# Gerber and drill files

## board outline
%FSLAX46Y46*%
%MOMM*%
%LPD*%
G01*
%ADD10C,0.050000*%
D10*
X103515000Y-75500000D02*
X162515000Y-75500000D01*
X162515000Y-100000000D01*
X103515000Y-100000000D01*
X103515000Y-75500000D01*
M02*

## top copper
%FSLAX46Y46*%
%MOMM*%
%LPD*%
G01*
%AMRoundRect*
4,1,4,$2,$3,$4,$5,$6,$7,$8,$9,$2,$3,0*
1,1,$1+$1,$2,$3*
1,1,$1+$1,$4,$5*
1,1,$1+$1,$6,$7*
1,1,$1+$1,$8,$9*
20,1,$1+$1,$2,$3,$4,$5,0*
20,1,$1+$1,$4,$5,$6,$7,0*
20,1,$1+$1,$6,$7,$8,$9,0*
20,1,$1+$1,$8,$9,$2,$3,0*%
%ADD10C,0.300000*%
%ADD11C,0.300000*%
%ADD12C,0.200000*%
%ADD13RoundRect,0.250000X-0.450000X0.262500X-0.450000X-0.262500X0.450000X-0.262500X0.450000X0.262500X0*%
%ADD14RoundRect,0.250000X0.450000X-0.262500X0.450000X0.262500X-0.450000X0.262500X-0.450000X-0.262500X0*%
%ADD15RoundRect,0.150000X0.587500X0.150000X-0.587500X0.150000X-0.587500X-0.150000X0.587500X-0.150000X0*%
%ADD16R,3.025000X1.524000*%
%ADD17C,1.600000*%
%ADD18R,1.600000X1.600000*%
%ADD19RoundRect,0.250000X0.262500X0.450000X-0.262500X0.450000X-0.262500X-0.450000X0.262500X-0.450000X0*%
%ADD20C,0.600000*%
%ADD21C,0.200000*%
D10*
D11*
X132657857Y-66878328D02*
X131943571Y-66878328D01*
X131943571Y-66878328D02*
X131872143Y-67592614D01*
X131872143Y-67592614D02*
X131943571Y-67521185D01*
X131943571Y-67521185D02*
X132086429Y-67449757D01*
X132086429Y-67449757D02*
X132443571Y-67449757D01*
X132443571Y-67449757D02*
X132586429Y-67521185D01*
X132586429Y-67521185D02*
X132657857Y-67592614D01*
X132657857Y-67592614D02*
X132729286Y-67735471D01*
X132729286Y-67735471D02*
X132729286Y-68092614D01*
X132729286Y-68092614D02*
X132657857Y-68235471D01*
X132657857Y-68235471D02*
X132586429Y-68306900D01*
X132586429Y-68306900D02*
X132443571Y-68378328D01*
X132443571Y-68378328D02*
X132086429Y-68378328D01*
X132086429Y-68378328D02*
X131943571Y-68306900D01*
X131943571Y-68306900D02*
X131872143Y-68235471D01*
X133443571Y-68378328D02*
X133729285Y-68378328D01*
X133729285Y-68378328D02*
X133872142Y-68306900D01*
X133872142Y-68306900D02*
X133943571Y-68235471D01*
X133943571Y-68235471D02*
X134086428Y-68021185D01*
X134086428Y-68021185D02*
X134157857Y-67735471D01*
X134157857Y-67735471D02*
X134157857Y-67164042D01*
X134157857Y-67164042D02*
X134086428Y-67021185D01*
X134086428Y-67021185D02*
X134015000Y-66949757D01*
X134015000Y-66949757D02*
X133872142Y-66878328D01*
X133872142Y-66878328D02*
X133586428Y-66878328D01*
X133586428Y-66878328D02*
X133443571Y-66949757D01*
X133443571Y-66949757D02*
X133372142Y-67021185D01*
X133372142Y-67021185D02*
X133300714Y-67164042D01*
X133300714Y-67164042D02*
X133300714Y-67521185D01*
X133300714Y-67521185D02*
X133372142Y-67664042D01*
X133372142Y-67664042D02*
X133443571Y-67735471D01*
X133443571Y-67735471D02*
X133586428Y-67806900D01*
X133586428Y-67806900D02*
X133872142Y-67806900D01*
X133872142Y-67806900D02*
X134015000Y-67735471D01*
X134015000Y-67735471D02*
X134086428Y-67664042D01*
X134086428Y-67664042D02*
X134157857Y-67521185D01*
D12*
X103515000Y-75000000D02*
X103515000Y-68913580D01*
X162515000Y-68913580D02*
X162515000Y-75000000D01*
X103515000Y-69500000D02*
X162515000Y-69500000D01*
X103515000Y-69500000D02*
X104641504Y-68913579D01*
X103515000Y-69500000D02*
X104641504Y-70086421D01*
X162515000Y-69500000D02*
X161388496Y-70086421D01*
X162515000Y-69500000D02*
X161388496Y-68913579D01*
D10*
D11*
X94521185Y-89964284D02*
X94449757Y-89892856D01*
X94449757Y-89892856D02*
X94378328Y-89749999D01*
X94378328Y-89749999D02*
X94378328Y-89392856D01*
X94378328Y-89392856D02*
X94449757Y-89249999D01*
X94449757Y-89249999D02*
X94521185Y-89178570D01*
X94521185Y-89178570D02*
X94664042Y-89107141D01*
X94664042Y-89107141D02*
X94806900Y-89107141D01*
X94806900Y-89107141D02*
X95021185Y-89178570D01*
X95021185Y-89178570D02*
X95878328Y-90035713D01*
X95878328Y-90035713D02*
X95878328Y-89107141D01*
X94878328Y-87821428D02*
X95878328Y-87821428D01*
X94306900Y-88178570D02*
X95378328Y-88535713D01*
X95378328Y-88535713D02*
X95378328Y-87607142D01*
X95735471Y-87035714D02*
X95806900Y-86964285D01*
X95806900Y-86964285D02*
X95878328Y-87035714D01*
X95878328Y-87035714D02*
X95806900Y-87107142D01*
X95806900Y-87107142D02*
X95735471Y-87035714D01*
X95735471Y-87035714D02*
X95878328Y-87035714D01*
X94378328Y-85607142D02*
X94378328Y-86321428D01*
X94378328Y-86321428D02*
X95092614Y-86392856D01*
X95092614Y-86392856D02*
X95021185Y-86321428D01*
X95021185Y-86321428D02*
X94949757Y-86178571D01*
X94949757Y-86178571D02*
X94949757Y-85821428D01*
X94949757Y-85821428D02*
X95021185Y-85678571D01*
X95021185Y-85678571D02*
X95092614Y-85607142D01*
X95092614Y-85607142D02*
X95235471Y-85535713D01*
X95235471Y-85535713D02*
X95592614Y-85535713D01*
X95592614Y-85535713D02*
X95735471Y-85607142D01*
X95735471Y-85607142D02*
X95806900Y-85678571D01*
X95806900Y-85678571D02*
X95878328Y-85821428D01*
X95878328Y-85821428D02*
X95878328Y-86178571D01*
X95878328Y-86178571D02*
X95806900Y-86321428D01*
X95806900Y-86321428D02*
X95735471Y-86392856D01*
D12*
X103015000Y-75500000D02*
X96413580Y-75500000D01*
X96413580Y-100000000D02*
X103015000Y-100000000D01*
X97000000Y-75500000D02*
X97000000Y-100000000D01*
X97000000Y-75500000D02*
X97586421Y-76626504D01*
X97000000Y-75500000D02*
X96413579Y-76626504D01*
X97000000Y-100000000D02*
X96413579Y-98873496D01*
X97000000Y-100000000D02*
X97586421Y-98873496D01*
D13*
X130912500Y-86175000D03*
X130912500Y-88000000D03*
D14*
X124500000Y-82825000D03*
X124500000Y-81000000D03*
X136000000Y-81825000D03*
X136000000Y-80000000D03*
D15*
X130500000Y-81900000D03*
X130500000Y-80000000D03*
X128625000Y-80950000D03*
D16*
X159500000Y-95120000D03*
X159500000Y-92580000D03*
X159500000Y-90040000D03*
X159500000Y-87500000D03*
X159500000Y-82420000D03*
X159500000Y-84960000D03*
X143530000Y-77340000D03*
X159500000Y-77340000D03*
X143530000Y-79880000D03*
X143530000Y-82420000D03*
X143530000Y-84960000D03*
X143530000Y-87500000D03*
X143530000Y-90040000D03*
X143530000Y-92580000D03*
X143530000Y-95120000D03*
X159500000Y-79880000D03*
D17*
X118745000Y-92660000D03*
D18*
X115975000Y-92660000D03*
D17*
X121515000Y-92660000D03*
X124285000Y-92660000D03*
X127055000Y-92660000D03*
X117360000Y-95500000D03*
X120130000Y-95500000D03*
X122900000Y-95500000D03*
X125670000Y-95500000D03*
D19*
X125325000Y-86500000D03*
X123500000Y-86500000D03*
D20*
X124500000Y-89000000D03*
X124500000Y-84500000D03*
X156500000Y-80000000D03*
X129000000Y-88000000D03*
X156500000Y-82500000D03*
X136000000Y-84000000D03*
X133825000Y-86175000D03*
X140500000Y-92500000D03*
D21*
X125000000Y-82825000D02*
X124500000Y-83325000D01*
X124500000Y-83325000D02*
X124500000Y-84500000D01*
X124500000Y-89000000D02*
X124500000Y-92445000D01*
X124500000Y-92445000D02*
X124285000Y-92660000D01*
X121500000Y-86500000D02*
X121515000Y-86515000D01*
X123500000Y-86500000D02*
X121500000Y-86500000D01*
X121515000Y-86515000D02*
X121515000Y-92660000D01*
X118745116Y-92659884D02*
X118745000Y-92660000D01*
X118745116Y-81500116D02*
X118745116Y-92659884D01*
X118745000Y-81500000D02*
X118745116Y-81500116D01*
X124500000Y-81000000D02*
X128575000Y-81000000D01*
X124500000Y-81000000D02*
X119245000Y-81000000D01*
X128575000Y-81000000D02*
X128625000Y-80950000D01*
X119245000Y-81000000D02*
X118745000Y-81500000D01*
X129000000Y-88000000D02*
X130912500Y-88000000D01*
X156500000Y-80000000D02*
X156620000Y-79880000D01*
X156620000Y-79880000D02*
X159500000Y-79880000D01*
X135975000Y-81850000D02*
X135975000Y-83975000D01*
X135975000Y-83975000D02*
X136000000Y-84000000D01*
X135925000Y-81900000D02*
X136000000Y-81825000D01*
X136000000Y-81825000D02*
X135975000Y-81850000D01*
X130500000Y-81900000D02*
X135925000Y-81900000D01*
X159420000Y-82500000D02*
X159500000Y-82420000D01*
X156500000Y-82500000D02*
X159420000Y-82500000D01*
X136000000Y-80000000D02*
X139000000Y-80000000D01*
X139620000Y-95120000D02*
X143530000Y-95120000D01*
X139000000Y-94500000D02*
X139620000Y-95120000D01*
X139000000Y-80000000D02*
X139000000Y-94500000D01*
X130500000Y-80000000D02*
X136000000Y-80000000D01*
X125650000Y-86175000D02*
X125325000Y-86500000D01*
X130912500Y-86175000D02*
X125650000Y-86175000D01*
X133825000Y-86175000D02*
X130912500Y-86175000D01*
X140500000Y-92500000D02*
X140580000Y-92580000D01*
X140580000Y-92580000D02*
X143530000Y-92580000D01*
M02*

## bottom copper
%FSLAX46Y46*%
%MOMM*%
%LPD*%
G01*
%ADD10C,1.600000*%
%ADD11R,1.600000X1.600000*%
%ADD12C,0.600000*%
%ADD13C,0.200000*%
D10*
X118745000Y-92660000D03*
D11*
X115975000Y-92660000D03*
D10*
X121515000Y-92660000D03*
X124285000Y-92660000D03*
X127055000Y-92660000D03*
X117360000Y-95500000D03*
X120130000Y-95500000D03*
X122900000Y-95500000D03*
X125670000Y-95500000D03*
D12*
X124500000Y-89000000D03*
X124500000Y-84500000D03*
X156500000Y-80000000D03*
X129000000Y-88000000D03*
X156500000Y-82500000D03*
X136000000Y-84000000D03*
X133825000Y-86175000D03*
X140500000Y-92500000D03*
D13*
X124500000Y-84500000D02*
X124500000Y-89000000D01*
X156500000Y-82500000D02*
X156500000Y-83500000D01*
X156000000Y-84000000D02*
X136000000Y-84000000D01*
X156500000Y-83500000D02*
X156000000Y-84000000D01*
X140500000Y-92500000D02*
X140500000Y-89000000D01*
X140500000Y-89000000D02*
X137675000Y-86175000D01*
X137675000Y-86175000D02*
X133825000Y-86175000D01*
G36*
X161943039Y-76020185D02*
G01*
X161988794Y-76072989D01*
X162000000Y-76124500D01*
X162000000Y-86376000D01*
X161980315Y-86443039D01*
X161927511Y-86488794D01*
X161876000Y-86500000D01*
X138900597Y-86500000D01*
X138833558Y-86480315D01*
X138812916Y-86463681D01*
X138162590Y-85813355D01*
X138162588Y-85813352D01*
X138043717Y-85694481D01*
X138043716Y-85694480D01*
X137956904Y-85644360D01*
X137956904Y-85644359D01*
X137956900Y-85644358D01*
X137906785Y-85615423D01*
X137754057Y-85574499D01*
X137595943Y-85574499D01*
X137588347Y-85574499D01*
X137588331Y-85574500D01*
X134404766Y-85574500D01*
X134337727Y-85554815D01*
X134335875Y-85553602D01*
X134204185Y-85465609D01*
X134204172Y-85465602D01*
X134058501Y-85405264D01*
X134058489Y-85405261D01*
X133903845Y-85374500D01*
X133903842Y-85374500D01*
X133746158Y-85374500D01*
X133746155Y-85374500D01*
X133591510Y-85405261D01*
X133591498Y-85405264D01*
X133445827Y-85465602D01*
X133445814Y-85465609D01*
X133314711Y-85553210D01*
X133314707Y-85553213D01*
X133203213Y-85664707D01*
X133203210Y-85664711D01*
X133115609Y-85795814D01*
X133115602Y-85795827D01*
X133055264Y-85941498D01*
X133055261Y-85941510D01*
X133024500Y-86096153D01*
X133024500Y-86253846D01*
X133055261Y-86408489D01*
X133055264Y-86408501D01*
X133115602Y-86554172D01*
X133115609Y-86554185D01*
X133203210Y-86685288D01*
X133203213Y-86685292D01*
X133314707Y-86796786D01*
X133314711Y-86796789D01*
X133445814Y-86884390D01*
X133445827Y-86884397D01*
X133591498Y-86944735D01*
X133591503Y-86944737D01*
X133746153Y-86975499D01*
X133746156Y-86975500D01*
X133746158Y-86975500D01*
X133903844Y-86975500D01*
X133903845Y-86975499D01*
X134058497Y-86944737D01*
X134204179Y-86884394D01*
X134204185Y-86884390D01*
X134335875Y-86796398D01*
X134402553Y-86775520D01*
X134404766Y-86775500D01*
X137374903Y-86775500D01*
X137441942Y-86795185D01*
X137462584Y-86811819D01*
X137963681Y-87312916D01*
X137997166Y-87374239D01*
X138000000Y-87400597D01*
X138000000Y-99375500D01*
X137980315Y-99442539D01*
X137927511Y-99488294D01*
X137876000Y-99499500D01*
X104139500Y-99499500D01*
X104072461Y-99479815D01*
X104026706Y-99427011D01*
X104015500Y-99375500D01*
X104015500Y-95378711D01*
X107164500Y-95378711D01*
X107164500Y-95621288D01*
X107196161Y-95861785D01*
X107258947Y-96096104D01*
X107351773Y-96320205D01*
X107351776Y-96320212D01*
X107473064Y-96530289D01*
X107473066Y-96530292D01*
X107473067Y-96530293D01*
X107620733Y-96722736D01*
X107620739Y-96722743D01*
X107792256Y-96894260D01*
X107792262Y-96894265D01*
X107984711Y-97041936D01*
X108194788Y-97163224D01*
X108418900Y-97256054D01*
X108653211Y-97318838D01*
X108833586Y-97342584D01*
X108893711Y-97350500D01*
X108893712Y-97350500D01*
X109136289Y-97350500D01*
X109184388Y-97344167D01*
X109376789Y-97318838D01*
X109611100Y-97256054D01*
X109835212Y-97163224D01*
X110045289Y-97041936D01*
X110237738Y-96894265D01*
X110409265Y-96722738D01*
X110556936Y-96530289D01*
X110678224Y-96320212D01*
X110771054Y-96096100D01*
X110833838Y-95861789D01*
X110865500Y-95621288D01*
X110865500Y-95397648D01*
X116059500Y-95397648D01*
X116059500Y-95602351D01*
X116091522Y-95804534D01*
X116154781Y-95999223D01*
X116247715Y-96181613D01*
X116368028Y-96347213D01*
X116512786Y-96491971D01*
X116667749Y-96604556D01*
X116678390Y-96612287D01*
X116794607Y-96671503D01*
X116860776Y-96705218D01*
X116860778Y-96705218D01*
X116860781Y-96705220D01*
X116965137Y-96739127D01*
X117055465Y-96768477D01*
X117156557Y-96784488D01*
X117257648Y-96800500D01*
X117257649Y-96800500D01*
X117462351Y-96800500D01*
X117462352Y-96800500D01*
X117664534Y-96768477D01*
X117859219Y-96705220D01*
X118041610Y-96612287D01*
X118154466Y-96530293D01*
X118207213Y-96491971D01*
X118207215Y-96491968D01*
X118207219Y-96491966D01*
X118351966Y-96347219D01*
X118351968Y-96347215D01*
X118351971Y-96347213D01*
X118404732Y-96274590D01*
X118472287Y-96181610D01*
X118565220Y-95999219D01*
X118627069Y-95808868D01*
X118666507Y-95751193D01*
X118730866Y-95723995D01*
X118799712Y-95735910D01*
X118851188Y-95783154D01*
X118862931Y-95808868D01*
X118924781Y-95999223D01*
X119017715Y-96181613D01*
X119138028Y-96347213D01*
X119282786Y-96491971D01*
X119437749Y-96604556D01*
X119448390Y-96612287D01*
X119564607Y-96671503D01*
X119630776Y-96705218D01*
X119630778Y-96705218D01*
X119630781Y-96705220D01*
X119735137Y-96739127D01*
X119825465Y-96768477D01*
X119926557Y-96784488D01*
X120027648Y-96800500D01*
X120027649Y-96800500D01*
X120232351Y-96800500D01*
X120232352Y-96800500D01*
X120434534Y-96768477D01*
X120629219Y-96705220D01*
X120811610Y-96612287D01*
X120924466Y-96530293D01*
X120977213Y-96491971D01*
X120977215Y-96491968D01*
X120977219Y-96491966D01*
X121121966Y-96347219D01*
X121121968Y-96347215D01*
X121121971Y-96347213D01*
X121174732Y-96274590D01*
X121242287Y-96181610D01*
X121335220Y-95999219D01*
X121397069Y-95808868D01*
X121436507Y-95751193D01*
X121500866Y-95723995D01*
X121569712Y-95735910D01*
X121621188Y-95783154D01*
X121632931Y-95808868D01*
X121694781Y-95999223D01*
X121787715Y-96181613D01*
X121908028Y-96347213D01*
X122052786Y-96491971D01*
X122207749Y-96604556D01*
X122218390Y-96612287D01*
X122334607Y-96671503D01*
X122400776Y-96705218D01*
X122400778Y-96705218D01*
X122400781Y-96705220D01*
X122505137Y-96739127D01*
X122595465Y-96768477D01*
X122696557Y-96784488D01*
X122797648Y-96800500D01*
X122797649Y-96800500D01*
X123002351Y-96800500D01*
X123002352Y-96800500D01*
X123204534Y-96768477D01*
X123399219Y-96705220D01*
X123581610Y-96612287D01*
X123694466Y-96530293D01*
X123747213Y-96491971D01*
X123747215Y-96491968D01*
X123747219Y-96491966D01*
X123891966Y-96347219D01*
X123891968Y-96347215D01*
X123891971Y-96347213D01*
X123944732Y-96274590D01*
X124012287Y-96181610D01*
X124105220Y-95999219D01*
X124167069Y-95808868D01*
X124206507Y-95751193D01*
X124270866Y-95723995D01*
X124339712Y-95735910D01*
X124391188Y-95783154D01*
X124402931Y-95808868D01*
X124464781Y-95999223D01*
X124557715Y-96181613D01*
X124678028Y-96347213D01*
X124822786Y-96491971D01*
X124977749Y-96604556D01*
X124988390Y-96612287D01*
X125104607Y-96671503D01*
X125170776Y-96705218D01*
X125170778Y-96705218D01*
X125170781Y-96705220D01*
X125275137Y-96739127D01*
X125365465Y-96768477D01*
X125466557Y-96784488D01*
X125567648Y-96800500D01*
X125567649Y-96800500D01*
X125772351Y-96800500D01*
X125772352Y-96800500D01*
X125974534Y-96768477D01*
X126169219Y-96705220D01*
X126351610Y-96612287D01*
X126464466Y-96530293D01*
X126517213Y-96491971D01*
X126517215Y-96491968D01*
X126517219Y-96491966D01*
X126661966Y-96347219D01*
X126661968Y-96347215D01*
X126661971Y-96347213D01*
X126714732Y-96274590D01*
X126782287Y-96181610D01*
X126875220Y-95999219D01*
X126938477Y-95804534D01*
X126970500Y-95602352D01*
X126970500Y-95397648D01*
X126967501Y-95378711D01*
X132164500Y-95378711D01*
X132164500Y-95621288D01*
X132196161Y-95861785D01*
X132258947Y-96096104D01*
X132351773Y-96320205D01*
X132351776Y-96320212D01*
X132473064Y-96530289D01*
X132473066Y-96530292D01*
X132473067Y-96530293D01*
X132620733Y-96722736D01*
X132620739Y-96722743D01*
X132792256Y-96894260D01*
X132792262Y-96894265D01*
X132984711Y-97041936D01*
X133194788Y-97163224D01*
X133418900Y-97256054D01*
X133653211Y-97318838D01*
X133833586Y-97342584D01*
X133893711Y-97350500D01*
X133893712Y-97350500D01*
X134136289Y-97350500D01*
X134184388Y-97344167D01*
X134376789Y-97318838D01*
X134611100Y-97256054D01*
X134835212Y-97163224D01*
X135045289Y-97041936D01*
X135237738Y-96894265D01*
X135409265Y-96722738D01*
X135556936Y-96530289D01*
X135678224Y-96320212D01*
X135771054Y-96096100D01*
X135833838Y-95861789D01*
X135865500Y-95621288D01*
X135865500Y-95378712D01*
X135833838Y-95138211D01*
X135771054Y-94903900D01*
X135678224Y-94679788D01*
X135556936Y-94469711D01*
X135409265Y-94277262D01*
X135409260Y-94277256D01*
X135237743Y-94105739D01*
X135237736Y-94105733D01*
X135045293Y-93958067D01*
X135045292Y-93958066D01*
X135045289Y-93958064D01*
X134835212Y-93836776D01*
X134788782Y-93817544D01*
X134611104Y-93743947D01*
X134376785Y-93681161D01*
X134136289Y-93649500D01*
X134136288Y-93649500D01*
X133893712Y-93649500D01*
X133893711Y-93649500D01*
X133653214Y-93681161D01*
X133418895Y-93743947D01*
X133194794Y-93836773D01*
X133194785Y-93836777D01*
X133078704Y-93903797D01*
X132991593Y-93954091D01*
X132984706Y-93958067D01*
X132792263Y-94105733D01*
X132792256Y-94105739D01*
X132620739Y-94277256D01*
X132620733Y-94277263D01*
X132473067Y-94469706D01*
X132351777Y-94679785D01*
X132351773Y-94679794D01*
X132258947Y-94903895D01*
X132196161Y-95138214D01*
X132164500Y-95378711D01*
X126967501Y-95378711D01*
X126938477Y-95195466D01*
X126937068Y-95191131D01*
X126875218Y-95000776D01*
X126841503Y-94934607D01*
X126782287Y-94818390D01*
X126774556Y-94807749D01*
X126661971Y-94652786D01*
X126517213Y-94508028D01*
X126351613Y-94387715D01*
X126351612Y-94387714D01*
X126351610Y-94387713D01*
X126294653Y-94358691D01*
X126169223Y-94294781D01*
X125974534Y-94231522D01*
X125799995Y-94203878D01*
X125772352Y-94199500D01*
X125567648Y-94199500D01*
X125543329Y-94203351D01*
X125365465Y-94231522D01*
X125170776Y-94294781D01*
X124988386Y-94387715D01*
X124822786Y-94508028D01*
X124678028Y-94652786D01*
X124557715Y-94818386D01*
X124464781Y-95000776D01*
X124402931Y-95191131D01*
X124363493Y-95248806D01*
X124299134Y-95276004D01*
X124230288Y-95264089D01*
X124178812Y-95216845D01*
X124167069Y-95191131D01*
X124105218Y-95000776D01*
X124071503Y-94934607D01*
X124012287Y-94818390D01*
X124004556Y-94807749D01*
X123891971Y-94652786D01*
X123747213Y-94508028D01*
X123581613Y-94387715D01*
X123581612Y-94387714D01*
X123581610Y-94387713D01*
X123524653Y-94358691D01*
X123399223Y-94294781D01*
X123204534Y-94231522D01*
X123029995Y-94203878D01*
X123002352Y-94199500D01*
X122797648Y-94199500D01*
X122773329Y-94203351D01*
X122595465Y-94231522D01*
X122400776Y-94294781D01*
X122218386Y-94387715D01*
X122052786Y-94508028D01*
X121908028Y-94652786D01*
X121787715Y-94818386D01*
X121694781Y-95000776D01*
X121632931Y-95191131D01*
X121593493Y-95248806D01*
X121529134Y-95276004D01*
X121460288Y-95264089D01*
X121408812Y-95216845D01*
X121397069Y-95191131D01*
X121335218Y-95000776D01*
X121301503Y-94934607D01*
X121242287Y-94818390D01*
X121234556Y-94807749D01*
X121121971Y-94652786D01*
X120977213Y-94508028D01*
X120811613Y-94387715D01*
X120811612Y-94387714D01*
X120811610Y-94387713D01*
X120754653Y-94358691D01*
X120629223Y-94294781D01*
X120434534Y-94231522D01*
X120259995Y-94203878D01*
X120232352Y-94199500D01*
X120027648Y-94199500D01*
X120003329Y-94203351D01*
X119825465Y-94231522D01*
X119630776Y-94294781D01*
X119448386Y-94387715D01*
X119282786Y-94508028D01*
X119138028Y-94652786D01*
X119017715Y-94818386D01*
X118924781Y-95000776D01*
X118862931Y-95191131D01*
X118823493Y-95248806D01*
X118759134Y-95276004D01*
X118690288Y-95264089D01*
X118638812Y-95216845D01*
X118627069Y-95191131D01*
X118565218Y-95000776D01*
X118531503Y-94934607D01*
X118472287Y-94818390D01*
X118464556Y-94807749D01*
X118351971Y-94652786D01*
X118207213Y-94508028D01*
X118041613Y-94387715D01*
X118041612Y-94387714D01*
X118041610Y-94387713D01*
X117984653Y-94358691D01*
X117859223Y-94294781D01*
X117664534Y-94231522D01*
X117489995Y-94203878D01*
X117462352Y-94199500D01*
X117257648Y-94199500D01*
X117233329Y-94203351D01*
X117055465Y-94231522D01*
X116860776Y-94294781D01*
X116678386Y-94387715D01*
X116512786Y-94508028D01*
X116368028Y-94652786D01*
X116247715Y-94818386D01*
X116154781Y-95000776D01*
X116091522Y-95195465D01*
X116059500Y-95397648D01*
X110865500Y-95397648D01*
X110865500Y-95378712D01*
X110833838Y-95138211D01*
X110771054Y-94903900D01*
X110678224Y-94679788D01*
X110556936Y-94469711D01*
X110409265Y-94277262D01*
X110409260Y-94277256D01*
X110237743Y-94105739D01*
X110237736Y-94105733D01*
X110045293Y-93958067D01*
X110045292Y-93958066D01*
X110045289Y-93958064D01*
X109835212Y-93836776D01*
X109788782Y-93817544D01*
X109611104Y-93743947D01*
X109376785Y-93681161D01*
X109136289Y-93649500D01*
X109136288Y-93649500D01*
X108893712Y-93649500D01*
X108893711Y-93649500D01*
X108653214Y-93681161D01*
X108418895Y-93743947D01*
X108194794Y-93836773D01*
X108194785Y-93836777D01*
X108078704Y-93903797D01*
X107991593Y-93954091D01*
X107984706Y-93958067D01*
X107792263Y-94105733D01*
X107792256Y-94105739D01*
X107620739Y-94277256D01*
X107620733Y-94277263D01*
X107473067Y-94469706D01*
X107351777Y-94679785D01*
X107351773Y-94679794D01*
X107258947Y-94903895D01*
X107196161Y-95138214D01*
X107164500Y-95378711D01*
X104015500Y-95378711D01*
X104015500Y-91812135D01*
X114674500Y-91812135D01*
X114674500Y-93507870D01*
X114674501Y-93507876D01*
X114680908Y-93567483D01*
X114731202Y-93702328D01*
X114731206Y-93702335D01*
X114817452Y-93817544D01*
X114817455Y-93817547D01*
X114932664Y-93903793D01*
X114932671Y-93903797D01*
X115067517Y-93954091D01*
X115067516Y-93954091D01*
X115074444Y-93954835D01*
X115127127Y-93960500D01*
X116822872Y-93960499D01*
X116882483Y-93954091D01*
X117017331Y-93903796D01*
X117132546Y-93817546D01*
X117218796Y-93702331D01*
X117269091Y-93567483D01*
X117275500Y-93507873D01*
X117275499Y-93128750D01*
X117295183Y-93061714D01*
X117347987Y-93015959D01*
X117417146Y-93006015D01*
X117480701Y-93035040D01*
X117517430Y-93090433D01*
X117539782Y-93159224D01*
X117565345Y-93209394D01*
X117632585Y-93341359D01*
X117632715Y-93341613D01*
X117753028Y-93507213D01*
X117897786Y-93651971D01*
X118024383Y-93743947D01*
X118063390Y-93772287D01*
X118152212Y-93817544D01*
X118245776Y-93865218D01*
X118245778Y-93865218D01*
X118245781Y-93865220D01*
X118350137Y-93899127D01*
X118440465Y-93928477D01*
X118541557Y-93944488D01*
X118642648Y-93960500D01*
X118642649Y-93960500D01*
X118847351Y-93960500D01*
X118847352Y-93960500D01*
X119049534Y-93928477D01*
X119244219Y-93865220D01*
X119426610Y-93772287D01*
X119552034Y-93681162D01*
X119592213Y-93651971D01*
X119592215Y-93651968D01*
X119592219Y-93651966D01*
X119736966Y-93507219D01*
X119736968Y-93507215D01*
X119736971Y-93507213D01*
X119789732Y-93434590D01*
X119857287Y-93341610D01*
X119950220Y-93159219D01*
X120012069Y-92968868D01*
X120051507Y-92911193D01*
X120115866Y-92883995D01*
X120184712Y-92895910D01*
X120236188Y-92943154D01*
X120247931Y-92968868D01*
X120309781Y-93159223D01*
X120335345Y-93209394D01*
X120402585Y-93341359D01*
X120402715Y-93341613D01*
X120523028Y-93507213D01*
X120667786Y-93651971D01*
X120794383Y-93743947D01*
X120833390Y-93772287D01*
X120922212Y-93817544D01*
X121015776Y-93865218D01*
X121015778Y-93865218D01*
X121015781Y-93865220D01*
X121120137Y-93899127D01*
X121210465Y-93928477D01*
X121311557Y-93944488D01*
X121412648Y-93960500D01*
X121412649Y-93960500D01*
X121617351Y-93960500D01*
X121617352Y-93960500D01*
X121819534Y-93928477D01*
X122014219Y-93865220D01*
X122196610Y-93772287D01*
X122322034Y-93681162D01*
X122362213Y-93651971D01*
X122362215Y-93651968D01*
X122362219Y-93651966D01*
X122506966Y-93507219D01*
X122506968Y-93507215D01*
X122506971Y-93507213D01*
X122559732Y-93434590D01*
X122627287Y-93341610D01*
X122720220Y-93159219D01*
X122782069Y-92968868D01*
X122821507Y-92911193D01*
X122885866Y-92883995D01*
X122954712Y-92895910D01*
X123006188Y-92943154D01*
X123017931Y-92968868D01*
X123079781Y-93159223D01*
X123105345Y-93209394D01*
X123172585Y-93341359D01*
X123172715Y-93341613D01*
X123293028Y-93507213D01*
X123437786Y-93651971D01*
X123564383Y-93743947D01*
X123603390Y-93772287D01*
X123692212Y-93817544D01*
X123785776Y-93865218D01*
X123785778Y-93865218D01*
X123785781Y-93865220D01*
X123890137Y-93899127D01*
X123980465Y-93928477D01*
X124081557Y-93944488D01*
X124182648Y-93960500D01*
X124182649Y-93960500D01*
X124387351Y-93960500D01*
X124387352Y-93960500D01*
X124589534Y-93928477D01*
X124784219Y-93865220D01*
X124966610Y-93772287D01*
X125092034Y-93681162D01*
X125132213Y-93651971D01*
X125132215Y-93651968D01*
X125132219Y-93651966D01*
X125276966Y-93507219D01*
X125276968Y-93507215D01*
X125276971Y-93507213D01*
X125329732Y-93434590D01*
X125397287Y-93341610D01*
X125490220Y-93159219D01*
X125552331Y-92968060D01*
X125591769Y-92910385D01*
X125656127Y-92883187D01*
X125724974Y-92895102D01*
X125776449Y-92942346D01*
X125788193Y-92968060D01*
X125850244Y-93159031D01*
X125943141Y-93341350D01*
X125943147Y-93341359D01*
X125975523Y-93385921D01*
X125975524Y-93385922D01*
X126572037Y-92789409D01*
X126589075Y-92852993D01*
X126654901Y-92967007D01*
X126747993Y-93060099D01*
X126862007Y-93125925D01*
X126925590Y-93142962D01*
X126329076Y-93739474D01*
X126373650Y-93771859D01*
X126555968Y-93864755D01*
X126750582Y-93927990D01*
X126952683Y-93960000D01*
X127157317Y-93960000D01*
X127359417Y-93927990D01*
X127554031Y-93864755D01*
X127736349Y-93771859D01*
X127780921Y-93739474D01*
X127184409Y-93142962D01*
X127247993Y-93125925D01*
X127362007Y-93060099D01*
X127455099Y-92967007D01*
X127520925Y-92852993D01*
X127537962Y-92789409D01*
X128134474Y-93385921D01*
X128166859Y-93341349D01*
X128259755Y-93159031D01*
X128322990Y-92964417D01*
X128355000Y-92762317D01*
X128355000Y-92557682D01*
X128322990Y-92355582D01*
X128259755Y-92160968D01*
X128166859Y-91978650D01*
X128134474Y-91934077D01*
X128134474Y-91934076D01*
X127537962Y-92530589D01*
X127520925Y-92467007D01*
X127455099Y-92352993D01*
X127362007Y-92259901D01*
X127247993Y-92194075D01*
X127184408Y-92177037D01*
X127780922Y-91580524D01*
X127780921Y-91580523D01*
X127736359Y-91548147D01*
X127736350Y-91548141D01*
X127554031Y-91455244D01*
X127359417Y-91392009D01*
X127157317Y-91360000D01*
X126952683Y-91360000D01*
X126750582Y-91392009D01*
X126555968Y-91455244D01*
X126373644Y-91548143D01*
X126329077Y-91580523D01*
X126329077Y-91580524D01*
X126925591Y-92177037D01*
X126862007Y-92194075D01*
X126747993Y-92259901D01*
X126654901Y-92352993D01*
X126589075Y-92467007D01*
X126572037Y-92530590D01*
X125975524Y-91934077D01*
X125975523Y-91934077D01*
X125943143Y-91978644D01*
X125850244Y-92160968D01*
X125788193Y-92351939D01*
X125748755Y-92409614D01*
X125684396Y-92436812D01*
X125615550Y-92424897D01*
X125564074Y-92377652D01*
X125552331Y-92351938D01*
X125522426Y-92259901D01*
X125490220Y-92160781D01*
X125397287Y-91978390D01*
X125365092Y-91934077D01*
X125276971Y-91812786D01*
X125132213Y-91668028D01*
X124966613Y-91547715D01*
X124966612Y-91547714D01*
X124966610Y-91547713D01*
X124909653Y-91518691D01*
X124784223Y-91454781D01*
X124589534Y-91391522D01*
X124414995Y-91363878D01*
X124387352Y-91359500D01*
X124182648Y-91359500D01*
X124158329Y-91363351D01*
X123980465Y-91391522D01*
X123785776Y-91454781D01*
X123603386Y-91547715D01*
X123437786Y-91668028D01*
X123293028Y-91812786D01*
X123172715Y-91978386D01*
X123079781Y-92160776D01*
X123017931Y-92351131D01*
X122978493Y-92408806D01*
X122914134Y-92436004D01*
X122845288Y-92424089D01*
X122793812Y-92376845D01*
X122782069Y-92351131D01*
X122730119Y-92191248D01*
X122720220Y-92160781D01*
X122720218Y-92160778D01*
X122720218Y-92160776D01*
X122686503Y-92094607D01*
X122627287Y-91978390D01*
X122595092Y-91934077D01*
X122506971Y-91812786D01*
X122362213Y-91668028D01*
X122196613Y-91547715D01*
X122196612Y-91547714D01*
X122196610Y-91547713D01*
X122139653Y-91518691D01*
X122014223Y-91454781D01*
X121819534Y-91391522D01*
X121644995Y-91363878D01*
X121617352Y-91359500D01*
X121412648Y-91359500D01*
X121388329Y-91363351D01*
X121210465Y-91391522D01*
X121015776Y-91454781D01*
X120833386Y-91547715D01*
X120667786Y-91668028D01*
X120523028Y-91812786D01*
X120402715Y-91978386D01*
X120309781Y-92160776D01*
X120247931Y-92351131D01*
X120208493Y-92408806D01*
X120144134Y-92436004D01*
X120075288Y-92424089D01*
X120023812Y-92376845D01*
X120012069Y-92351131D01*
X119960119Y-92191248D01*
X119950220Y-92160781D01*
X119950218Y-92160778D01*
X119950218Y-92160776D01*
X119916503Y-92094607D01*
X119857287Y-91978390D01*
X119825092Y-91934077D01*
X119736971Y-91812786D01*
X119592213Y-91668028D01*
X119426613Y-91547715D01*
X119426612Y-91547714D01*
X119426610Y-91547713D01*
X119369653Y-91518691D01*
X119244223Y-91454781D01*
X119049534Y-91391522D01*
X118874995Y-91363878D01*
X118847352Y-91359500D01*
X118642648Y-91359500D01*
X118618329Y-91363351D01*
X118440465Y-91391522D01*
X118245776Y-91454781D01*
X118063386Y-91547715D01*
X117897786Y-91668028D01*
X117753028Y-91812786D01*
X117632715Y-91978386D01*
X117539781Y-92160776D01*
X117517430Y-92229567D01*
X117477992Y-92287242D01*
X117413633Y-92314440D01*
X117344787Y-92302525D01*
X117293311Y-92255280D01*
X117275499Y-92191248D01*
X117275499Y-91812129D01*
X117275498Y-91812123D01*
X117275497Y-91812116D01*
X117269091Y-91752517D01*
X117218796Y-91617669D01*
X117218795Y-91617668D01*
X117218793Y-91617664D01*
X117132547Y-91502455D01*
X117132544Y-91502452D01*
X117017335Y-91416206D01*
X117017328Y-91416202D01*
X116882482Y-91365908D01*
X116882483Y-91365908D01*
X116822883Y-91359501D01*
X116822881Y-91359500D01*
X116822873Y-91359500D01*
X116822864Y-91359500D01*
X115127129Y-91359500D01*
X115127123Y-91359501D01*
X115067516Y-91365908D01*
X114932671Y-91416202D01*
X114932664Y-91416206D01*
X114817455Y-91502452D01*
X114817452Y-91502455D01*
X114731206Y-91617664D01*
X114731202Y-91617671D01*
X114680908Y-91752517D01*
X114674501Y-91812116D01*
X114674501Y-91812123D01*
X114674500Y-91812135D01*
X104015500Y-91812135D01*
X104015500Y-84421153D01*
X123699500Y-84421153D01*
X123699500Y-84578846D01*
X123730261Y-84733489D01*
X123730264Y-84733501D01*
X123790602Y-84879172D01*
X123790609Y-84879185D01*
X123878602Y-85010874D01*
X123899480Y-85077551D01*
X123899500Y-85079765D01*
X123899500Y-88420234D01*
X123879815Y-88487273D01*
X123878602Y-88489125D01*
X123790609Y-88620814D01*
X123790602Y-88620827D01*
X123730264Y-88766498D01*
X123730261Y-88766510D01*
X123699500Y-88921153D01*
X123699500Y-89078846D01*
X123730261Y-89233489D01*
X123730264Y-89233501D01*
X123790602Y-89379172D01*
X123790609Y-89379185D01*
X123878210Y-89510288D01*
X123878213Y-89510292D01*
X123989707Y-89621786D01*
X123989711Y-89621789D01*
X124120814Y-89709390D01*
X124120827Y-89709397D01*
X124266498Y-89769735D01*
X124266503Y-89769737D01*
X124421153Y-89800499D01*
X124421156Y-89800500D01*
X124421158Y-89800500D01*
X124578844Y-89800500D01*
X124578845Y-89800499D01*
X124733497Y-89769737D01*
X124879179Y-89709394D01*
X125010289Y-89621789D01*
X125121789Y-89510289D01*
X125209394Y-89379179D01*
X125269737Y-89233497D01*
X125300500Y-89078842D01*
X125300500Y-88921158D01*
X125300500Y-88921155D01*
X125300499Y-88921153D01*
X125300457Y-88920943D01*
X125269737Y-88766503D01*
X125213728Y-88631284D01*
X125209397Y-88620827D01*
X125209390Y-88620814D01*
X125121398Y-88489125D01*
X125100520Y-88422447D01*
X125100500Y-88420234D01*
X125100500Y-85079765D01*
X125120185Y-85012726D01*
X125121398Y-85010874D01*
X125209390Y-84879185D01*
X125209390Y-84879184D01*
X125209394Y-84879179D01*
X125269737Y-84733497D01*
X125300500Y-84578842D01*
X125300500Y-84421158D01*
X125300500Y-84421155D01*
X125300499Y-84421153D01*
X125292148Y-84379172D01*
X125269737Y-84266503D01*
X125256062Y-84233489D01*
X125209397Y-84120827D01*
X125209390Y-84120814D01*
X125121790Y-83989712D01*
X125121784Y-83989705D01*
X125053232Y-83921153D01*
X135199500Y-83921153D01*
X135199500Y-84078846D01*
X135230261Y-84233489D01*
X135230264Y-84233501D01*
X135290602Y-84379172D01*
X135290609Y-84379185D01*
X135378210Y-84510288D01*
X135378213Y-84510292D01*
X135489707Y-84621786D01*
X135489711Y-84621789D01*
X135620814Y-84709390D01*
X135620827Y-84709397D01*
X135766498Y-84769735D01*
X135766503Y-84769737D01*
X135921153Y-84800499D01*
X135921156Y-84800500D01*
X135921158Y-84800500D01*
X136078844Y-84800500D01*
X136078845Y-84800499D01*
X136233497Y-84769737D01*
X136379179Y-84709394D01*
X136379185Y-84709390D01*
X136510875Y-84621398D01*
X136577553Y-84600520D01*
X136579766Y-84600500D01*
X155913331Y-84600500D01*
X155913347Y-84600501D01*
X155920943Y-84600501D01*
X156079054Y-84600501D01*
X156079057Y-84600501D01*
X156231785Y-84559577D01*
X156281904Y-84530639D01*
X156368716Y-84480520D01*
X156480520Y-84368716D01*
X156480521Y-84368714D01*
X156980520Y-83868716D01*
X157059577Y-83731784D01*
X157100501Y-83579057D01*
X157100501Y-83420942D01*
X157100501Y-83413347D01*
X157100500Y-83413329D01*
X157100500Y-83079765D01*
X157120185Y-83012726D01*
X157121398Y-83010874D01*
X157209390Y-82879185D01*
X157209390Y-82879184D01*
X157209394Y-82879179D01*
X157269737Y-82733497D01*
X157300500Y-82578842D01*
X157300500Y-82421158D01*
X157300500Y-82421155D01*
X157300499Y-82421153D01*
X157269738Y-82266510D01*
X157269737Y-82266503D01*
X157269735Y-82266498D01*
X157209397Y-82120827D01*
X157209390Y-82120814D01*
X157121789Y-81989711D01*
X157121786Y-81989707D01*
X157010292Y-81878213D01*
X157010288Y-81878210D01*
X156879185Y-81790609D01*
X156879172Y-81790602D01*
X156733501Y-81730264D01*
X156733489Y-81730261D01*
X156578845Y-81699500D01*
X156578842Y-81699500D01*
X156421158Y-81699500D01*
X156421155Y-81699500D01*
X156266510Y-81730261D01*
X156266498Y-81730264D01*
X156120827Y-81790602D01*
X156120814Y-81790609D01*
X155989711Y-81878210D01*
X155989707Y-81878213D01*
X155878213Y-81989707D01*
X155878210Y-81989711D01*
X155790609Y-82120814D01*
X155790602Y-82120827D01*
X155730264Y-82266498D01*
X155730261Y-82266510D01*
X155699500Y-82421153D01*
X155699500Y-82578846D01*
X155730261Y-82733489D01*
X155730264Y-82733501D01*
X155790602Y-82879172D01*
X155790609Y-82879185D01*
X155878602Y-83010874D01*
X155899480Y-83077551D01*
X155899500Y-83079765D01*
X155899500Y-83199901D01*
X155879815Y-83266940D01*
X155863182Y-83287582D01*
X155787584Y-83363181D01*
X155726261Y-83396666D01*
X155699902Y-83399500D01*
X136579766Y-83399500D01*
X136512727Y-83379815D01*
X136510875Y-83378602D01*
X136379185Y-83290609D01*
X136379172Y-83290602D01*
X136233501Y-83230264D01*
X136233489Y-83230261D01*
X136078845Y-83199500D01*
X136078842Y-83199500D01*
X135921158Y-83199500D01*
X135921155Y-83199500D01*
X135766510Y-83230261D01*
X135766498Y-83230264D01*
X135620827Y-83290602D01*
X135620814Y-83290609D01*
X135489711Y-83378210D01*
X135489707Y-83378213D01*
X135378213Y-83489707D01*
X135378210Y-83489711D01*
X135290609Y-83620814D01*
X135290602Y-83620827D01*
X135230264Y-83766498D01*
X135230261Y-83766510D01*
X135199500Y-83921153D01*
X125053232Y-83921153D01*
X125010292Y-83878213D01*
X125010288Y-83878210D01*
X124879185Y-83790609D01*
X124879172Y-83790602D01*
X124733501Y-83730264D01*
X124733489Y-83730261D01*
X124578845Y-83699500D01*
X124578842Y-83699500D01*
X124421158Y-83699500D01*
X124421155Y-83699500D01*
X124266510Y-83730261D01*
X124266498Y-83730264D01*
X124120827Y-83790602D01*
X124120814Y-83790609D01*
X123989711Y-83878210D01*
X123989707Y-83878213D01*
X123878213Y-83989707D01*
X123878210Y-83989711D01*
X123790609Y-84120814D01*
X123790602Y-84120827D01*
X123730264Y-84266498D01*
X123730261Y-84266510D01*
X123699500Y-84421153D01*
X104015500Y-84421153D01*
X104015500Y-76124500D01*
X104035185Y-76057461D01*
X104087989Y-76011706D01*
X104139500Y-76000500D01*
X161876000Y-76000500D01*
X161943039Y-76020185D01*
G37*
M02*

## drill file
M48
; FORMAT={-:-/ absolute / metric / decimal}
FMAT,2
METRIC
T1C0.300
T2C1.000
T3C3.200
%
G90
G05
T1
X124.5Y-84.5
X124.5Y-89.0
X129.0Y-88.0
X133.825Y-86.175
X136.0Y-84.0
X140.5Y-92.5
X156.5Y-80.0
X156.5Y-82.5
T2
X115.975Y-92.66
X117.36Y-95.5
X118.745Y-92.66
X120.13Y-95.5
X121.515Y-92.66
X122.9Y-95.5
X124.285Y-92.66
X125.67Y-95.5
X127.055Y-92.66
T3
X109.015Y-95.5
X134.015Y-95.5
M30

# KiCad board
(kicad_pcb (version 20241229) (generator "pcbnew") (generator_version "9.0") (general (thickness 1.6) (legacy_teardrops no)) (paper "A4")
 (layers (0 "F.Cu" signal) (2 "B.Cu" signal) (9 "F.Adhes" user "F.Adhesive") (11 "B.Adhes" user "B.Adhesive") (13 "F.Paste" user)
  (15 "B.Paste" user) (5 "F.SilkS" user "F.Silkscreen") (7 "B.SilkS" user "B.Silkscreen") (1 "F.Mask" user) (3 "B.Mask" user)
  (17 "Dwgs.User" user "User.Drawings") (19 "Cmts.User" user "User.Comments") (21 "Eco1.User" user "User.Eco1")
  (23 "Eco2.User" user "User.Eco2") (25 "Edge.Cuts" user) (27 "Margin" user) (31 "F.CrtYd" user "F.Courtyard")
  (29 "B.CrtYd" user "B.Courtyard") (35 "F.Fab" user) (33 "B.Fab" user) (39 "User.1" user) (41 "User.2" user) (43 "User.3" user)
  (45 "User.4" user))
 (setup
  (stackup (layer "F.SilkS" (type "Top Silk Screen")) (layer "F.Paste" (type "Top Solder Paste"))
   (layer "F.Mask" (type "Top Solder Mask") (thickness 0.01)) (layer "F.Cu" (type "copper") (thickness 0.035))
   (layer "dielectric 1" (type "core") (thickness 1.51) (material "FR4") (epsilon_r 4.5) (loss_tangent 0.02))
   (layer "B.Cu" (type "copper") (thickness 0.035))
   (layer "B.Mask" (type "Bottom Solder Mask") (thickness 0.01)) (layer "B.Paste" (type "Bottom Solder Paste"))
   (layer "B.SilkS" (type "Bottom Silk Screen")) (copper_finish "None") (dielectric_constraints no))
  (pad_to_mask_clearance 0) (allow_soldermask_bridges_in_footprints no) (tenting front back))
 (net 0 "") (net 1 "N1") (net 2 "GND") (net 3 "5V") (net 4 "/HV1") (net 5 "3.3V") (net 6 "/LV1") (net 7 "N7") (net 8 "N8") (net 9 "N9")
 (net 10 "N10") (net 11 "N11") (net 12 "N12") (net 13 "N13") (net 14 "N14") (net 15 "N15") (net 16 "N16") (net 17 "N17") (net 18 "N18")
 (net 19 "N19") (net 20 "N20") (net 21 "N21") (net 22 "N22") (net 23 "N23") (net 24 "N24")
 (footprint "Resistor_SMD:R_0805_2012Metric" (layer "F.Cu") (at 130.9125 87.0875 -90)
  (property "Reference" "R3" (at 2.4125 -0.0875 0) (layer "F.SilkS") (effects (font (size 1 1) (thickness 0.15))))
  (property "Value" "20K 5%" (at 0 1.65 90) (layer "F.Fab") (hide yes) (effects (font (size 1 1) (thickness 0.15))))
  (pad "1" smd roundrect (at -0.9125 0 270) (size 1.025 1.4) (layers "F.Cu" "F.Mask" "F.Paste") (roundrect_rratio 0.243902) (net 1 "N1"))
  (pad "2" smd roundrect (at 0.9125 0 270) (size 1.025 1.4) (layers "F.Cu" "F.Mask" "F.Paste") (roundrect_rratio 0.243902) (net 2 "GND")))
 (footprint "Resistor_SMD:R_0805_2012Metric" (layer "F.Cu") (at 124.5 81.9125 90)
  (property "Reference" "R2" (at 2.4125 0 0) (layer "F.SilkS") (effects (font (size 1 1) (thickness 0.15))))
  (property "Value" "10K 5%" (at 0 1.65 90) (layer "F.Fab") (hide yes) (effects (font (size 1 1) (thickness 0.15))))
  (pad "1" smd roundrect (at -0.9125 0 90) (size 1.025 1.4) (layers "F.Cu" "F.Mask" "F.Paste") (roundrect_rratio 0.243902) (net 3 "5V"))
  (pad "2" smd roundrect (at 0.9125 0 90) (size 1.025 1.4) (layers "F.Cu" "F.Mask" "F.Paste") (roundrect_rratio 0.243902) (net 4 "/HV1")))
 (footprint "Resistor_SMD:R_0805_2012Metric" (layer "F.Cu") (at 136 80.9125 90)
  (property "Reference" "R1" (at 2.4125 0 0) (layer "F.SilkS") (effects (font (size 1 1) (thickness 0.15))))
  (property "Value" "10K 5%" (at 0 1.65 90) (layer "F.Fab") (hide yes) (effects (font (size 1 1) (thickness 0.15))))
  (pad "1" smd roundrect (at -0.9125 0 90) (size 1.025 1.4) (layers "F.Cu" "F.Mask" "F.Paste") (roundrect_rratio 0.243902) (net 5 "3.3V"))
  (pad "2" smd roundrect (at 0.9125 0 90) (size 1.025 1.4) (layers "F.Cu" "F.Mask" "F.Paste") (roundrect_rratio 0.243902) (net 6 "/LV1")))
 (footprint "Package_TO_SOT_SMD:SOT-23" (layer "F.Cu") (at 129.5625 80.95 180)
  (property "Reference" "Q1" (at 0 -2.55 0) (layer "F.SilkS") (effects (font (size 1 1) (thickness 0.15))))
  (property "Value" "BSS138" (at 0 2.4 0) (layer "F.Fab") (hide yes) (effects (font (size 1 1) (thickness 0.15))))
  (pad "1" smd roundrect (at -0.9375 -0.95 180) (size 1.475 0.6) (layers "F.Cu" "F.Mask" "F.Paste") (roundrect_rratio 0.25) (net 5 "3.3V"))
  (pad "2" smd roundrect (at -0.9375 0.95 180) (size 1.475 0.6) (layers "F.Cu" "F.Mask" "F.Paste") (roundrect_rratio 0.25) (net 6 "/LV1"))
  (pad "3" smd roundrect (at 0.9375 0 180) (size 1.475 0.6) (layers "F.Cu" "F.Mask" "F.Paste") (roundrect_rratio 0.25) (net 4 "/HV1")))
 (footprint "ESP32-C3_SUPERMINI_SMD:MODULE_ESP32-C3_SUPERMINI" (layer "F.Cu") (at 151.515 87.24)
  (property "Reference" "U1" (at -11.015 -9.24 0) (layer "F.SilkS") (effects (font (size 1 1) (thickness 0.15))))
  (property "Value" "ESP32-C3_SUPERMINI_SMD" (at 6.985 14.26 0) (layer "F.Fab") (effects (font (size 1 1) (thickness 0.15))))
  (pad "0" smd rect (at 7.985 7.88) (size 3.025 1.524) (layers "F.Cu" "F.Mask" "F.Paste") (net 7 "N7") (solder_mask_margin 0.102))
  (pad "1" smd rect (at 7.985 5.34) (size 3.025 1.524) (layers "F.Cu" "F.Mask" "F.Paste") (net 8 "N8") (solder_mask_margin 0.102))
  (pad "2" smd rect (at 7.985 2.8) (size 3.025 1.524) (layers "F.Cu" "F.Mask" "F.Paste") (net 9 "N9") (solder_mask_margin 0.102))
  (pad "3" smd rect (at 7.985 0.26) (size 3.025 1.524) (layers "F.Cu" "F.Mask" "F.Paste") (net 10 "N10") (solder_mask_margin 0.102))
  (pad "3.3" smd rect (at 7.985 -4.82) (size 3.025 1.524) (layers "F.Cu" "F.Mask" "F.Paste") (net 5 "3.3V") (solder_mask_margin 0.102))
  (pad "4" smd rect (at 7.985 -2.28) (size 3.025 1.524) (layers "F.Cu" "F.Mask" "F.Paste") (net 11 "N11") (solder_mask_margin 0.102))
  (pad "5" smd rect (at -7.985 -9.9) (size 3.025 1.524) (layers "F.Cu" "F.Mask" "F.Paste") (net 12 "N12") (solder_mask_margin 0.102))
  (pad "5V" smd rect (at 7.985 -9.9) (size 3.025 1.524) (layers "F.Cu" "F.Mask" "F.Paste") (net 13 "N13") (solder_mask_margin 0.102))
  (pad "6" smd rect (at -7.985 -7.36) (size 3.025 1.524) (layers "F.Cu" "F.Mask" "F.Paste") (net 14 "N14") (solder_mask_margin 0.102))
  (pad "7" smd rect (at -7.985 -4.82) (size 3.025 1.524) (layers "F.Cu" "F.Mask" "F.Paste") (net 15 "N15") (solder_mask_margin 0.102))
  (pad "8" smd rect (at -7.985 -2.28) (size 3.025 1.524) (layers "F.Cu" "F.Mask" "F.Paste") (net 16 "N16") (solder_mask_margin 0.102))
  (pad "9" smd rect (at -7.985 0.26) (size 3.025 1.524) (layers "F.Cu" "F.Mask" "F.Paste") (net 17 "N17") (solder_mask_margin 0.102))
  (pad "10" smd rect (at -7.985 2.8) (size 3.025 1.524) (layers "F.Cu" "F.Mask" "F.Paste") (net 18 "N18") (solder_mask_margin 0.102))
  (pad "20" smd rect (at -7.985 5.34) (size 3.025 1.524) (layers "F.Cu" "F.Mask" "F.Paste") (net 1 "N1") (solder_mask_margin 0.102))
  (pad "21" smd rect (at -7.985 7.88) (size 3.025 1.524) (layers "F.Cu" "F.Mask" "F.Paste") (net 6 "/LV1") (solder_mask_margin 0.102))
  (pad "G" smd rect (at 7.985 -7.36) (size 3.025 1.524) (layers "F.Cu" "F.Mask" "F.Paste") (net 2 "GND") (solder_mask_margin 0.102)))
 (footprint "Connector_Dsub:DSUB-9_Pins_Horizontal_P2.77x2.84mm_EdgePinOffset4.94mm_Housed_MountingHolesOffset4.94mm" (layer "F.Cu")
  (at 115.975 92.66)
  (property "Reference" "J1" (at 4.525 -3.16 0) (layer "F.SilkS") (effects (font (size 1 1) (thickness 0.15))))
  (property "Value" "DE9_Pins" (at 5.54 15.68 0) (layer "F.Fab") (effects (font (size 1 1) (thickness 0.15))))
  (pad "" np_thru_hole circle (at -6.96 2.84) (size 4 4) (drill 3.2) (layers "*.Mask") (zone_connect 0))
  (pad "" thru_hole circle (at 2.77 0) (size 1.6 1.6) (drill 1) (layers "*.Cu" "*.Mask") (remove_unused_layers no))
  (pad "" np_thru_hole circle (at 18.04 2.84) (size 4 4) (drill 3.2) (layers "*.Mask") (zone_connect 0))
  (pad "1" thru_hole rect (at 0 0) (size 1.6 1.6) (drill 1) (layers "*.Cu" "*.Mask") (remove_unused_layers no) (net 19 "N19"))
  (pad "3" thru_hole circle (at 5.54 0) (size 1.6 1.6) (drill 1) (layers "*.Cu" "*.Mask") (remove_unused_layers no) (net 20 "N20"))
  (pad "4" thru_hole circle (at 8.31 0) (size 1.6 1.6) (drill 1) (layers "*.Cu" "*.Mask") (remove_unused_layers no) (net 3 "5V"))
  (pad "5" thru_hole circle (at 11.08 0) (size 1.6 1.6) (drill 1) (layers "*.Cu" "*.Mask") (remove_unused_layers no) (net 2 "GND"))
  (pad "6" thru_hole circle (at 1.385 2.84) (size 1.6 1.6) (drill 1) (layers "*.Cu" "*.Mask") (remove_unused_layers no) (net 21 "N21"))
  (pad "7" thru_hole circle (at 4.155 2.84) (size 1.6 1.6) (drill 1) (layers "*.Cu" "*.Mask") (remove_unused_layers no) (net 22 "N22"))
  (pad "8" thru_hole circle (at 6.925 2.84) (size 1.6 1.6) (drill 1) (layers "*.Cu" "*.Mask") (remove_unused_layers no) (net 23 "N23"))
  (pad "9" thru_hole circle (at 9.695 2.84) (size 1.6 1.6) (drill 1) (layers "*.Cu" "*.Mask") (remove_unused_layers no) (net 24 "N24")))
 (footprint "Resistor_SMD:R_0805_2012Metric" (layer "F.Cu") (at 124.4125 86.5 180)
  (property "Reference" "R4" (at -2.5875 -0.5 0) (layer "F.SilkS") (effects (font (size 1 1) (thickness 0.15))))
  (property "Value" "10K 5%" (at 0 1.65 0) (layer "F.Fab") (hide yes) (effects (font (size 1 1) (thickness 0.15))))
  (pad "1" smd roundrect (at -0.9125 0 180) (size 1.025 1.4) (layers "F.Cu" "F.Mask" "F.Paste") (roundrect_rratio 0.243902) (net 1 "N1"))
  (pad "2" smd roundrect (at 0.9125 0 180) (size 1.025 1.4) (layers "F.Cu" "F.Mask" "F.Paste") (roundrect_rratio 0.243902) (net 20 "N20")))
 (gr_rect (start 103.515 75.5) (end 162.515 100) (stroke (width 0.05) (type default)) (fill no) (layer "Edge.Cuts"))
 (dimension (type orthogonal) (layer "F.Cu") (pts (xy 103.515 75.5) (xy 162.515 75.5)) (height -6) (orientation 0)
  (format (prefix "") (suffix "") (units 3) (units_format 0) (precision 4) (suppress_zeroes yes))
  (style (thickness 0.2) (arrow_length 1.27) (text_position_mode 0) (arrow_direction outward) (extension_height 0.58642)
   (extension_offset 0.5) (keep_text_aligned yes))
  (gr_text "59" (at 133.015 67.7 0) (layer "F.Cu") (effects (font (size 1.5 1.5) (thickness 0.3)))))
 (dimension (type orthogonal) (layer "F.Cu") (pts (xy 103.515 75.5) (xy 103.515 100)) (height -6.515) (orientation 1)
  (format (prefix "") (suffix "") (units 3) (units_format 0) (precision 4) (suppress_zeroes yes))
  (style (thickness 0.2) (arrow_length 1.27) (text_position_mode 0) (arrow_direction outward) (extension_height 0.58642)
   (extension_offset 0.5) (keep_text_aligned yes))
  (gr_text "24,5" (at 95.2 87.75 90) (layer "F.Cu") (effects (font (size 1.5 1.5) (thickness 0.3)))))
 (segment (start 125 82.825) (end 124.5 83.325) (width 0.2) (layer "F.Cu") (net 3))
 (segment (start 124.5 83.325) (end 124.5 84.5) (width 0.2) (layer "F.Cu") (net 3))
 (segment (start 124.5 89) (end 124.5 92.445) (width 0.2) (layer "F.Cu") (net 3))
 (segment (start 124.5 92.445) (end 124.285 92.66) (width 0.2) (layer "F.Cu") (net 3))
 (via (at 124.5 89) (size 0.6) (drill 0.3) (layers "F.Cu" "B.Cu") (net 3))
 (via (at 124.5 84.5) (size 0.6) (drill 0.3) (layers "F.Cu" "B.Cu") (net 3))
 (segment (start 124.5 84.5) (end 124.5 89) (width 0.2) (layer "B.Cu") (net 3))
 (segment (start 121.5 86.5) (end 121.515 86.515) (width 0.2) (layer "F.Cu") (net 20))
 (segment (start 123.5 86.5) (end 121.5 86.5) (width 0.2) (layer "F.Cu") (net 20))
 (segment (start 121.515 86.515) (end 121.515 92.66) (width 0.2) (layer "F.Cu") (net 20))
 (segment (start 118.745116 92.659884) (end 118.745 92.66) (width 0.2) (layer "F.Cu") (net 4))
 (segment (start 118.745116 81.500116) (end 118.745116 92.659884) (width 0.2) (layer "F.Cu") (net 4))
 (segment (start 118.745 81.5) (end 118.745116 81.500116) (width 0.2) (layer "F.Cu") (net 4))
 (segment (start 124.5 81) (end 128.575 81) (width 0.2) (layer "F.Cu") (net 4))
 (segment (start 124.5 81) (end 119.245 81) (width 0.2) (layer "F.Cu") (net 4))
 (segment (start 128.575 81) (end 128.625 80.95) (width 0.2) (layer "F.Cu") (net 4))
 (segment (start 119.245 81) (end 118.745 81.5) (width 0.2) (layer "F.Cu") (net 4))
 (segment (start 129 88) (end 130.9125 88) (width 0.2) (layer "F.Cu") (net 2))
 (segment (start 156.5 80) (end 156.62 79.88) (width 0.2) (layer "F.Cu") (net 2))
 (segment (start 156.62 79.88) (end 159.5 79.88) (width 0.2) (layer "F.Cu") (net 2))
 (via (at 156.5 80) (size 0.6) (drill 0.3) (layers "F.Cu" "B.Cu") (free yes) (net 2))
 (via (at 129 88) (size 0.6) (drill 0.3) (layers "F.Cu" "B.Cu") (free yes) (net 2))
 (segment (start 135.975 81.85) (end 135.975 83.975) (width 0.2) (layer "F.Cu") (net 5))
 (segment (start 135.975 83.975) (end 136 84) (width 0.2) (layer "F.Cu") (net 5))
 (segment (start 135.925 81.9) (end 136 81.825) (width 0.2) (layer "F.Cu") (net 5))
 (segment (start 136 81.825) (end 135.975 81.85) (width 0.2) (layer "F.Cu") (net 5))
 (segment (start 130.5 81.9) (end 135.925 81.9) (width 0.2) (layer "F.Cu") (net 5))
 (segment (start 159.42 82.5) (end 159.5 82.42) (width 0.2) (layer "F.Cu") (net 5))
 (segment (start 156.5 82.5) (end 159.42 82.5) (width 0.2) (layer "F.Cu") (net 5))
 (via (at 156.5 82.5) (size 0.6) (drill 0.3) (layers "F.Cu" "B.Cu") (free yes) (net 5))
 (via (at 136 84) (size 0.6) (drill 0.3) (layers "F.Cu" "B.Cu") (free yes) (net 5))
 (segment (start 156.5 82.5) (end 156.5 83.5) (width 0.2) (layer "B.Cu") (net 5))
 (segment (start 156 84) (end 136 84) (width 0.2) (layer "B.Cu") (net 5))
 (segment (start 156.5 83.5) (end 156 84) (width 0.2) (layer "B.Cu") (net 5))
 (segment (start 136 80) (end 139 80) (width 0.2) (layer "F.Cu") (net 6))
 (segment (start 139.62 95.12) (end 143.53 95.12) (width 0.2) (layer "F.Cu") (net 6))
 (segment (start 139 94.5) (end 139.62 95.12) (width 0.2) (layer "F.Cu") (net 6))
 (segment (start 139 80) (end 139 94.5) (width 0.2) (layer "F.Cu") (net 6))
 (segment (start 130.5 80) (end 136 80) (width 0.2) (layer "F.Cu") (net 6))
 (segment (start 125.65 86.175) (end 125.325 86.5) (width 0.2) (layer "F.Cu") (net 1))
 (segment (start 130.9125 86.175) (end 125.65 86.175) (width 0.2) (layer "F.Cu") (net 1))
 (segment (start 133.825 86.175) (end 130.9125 86.175) (width 0.2) (layer "F.Cu") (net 1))
 (segment (start 140.5 92.5) (end 140.58 92.58) (width 0.2) (layer "F.Cu") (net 1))
 (segment (start 140.58 92.58) (end 143.53 92.58) (width 0.2) (layer "F.Cu") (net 1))
 (via (at 133.825 86.175) (size 0.6) (drill 0.3) (layers "F.Cu" "B.Cu") (free yes) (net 1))
 (via (at 140.5 92.5) (size 0.6) (drill 0.3) (layers "F.Cu" "B.Cu") (free yes) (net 1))
 (segment (start 140.5 92.5) (end 140.5 89) (width 0.2) (layer "B.Cu") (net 1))
 (segment (start 140.5 89) (end 137.675 86.175) (width 0.2) (layer "B.Cu") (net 1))
 (segment (start 137.675 86.175) (end 133.825 86.175) (width 0.2) (layer "B.Cu") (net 1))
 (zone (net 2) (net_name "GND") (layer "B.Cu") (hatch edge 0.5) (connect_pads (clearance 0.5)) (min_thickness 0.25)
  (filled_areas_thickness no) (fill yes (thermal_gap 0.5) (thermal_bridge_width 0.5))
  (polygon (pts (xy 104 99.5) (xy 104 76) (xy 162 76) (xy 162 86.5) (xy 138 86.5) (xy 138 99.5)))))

